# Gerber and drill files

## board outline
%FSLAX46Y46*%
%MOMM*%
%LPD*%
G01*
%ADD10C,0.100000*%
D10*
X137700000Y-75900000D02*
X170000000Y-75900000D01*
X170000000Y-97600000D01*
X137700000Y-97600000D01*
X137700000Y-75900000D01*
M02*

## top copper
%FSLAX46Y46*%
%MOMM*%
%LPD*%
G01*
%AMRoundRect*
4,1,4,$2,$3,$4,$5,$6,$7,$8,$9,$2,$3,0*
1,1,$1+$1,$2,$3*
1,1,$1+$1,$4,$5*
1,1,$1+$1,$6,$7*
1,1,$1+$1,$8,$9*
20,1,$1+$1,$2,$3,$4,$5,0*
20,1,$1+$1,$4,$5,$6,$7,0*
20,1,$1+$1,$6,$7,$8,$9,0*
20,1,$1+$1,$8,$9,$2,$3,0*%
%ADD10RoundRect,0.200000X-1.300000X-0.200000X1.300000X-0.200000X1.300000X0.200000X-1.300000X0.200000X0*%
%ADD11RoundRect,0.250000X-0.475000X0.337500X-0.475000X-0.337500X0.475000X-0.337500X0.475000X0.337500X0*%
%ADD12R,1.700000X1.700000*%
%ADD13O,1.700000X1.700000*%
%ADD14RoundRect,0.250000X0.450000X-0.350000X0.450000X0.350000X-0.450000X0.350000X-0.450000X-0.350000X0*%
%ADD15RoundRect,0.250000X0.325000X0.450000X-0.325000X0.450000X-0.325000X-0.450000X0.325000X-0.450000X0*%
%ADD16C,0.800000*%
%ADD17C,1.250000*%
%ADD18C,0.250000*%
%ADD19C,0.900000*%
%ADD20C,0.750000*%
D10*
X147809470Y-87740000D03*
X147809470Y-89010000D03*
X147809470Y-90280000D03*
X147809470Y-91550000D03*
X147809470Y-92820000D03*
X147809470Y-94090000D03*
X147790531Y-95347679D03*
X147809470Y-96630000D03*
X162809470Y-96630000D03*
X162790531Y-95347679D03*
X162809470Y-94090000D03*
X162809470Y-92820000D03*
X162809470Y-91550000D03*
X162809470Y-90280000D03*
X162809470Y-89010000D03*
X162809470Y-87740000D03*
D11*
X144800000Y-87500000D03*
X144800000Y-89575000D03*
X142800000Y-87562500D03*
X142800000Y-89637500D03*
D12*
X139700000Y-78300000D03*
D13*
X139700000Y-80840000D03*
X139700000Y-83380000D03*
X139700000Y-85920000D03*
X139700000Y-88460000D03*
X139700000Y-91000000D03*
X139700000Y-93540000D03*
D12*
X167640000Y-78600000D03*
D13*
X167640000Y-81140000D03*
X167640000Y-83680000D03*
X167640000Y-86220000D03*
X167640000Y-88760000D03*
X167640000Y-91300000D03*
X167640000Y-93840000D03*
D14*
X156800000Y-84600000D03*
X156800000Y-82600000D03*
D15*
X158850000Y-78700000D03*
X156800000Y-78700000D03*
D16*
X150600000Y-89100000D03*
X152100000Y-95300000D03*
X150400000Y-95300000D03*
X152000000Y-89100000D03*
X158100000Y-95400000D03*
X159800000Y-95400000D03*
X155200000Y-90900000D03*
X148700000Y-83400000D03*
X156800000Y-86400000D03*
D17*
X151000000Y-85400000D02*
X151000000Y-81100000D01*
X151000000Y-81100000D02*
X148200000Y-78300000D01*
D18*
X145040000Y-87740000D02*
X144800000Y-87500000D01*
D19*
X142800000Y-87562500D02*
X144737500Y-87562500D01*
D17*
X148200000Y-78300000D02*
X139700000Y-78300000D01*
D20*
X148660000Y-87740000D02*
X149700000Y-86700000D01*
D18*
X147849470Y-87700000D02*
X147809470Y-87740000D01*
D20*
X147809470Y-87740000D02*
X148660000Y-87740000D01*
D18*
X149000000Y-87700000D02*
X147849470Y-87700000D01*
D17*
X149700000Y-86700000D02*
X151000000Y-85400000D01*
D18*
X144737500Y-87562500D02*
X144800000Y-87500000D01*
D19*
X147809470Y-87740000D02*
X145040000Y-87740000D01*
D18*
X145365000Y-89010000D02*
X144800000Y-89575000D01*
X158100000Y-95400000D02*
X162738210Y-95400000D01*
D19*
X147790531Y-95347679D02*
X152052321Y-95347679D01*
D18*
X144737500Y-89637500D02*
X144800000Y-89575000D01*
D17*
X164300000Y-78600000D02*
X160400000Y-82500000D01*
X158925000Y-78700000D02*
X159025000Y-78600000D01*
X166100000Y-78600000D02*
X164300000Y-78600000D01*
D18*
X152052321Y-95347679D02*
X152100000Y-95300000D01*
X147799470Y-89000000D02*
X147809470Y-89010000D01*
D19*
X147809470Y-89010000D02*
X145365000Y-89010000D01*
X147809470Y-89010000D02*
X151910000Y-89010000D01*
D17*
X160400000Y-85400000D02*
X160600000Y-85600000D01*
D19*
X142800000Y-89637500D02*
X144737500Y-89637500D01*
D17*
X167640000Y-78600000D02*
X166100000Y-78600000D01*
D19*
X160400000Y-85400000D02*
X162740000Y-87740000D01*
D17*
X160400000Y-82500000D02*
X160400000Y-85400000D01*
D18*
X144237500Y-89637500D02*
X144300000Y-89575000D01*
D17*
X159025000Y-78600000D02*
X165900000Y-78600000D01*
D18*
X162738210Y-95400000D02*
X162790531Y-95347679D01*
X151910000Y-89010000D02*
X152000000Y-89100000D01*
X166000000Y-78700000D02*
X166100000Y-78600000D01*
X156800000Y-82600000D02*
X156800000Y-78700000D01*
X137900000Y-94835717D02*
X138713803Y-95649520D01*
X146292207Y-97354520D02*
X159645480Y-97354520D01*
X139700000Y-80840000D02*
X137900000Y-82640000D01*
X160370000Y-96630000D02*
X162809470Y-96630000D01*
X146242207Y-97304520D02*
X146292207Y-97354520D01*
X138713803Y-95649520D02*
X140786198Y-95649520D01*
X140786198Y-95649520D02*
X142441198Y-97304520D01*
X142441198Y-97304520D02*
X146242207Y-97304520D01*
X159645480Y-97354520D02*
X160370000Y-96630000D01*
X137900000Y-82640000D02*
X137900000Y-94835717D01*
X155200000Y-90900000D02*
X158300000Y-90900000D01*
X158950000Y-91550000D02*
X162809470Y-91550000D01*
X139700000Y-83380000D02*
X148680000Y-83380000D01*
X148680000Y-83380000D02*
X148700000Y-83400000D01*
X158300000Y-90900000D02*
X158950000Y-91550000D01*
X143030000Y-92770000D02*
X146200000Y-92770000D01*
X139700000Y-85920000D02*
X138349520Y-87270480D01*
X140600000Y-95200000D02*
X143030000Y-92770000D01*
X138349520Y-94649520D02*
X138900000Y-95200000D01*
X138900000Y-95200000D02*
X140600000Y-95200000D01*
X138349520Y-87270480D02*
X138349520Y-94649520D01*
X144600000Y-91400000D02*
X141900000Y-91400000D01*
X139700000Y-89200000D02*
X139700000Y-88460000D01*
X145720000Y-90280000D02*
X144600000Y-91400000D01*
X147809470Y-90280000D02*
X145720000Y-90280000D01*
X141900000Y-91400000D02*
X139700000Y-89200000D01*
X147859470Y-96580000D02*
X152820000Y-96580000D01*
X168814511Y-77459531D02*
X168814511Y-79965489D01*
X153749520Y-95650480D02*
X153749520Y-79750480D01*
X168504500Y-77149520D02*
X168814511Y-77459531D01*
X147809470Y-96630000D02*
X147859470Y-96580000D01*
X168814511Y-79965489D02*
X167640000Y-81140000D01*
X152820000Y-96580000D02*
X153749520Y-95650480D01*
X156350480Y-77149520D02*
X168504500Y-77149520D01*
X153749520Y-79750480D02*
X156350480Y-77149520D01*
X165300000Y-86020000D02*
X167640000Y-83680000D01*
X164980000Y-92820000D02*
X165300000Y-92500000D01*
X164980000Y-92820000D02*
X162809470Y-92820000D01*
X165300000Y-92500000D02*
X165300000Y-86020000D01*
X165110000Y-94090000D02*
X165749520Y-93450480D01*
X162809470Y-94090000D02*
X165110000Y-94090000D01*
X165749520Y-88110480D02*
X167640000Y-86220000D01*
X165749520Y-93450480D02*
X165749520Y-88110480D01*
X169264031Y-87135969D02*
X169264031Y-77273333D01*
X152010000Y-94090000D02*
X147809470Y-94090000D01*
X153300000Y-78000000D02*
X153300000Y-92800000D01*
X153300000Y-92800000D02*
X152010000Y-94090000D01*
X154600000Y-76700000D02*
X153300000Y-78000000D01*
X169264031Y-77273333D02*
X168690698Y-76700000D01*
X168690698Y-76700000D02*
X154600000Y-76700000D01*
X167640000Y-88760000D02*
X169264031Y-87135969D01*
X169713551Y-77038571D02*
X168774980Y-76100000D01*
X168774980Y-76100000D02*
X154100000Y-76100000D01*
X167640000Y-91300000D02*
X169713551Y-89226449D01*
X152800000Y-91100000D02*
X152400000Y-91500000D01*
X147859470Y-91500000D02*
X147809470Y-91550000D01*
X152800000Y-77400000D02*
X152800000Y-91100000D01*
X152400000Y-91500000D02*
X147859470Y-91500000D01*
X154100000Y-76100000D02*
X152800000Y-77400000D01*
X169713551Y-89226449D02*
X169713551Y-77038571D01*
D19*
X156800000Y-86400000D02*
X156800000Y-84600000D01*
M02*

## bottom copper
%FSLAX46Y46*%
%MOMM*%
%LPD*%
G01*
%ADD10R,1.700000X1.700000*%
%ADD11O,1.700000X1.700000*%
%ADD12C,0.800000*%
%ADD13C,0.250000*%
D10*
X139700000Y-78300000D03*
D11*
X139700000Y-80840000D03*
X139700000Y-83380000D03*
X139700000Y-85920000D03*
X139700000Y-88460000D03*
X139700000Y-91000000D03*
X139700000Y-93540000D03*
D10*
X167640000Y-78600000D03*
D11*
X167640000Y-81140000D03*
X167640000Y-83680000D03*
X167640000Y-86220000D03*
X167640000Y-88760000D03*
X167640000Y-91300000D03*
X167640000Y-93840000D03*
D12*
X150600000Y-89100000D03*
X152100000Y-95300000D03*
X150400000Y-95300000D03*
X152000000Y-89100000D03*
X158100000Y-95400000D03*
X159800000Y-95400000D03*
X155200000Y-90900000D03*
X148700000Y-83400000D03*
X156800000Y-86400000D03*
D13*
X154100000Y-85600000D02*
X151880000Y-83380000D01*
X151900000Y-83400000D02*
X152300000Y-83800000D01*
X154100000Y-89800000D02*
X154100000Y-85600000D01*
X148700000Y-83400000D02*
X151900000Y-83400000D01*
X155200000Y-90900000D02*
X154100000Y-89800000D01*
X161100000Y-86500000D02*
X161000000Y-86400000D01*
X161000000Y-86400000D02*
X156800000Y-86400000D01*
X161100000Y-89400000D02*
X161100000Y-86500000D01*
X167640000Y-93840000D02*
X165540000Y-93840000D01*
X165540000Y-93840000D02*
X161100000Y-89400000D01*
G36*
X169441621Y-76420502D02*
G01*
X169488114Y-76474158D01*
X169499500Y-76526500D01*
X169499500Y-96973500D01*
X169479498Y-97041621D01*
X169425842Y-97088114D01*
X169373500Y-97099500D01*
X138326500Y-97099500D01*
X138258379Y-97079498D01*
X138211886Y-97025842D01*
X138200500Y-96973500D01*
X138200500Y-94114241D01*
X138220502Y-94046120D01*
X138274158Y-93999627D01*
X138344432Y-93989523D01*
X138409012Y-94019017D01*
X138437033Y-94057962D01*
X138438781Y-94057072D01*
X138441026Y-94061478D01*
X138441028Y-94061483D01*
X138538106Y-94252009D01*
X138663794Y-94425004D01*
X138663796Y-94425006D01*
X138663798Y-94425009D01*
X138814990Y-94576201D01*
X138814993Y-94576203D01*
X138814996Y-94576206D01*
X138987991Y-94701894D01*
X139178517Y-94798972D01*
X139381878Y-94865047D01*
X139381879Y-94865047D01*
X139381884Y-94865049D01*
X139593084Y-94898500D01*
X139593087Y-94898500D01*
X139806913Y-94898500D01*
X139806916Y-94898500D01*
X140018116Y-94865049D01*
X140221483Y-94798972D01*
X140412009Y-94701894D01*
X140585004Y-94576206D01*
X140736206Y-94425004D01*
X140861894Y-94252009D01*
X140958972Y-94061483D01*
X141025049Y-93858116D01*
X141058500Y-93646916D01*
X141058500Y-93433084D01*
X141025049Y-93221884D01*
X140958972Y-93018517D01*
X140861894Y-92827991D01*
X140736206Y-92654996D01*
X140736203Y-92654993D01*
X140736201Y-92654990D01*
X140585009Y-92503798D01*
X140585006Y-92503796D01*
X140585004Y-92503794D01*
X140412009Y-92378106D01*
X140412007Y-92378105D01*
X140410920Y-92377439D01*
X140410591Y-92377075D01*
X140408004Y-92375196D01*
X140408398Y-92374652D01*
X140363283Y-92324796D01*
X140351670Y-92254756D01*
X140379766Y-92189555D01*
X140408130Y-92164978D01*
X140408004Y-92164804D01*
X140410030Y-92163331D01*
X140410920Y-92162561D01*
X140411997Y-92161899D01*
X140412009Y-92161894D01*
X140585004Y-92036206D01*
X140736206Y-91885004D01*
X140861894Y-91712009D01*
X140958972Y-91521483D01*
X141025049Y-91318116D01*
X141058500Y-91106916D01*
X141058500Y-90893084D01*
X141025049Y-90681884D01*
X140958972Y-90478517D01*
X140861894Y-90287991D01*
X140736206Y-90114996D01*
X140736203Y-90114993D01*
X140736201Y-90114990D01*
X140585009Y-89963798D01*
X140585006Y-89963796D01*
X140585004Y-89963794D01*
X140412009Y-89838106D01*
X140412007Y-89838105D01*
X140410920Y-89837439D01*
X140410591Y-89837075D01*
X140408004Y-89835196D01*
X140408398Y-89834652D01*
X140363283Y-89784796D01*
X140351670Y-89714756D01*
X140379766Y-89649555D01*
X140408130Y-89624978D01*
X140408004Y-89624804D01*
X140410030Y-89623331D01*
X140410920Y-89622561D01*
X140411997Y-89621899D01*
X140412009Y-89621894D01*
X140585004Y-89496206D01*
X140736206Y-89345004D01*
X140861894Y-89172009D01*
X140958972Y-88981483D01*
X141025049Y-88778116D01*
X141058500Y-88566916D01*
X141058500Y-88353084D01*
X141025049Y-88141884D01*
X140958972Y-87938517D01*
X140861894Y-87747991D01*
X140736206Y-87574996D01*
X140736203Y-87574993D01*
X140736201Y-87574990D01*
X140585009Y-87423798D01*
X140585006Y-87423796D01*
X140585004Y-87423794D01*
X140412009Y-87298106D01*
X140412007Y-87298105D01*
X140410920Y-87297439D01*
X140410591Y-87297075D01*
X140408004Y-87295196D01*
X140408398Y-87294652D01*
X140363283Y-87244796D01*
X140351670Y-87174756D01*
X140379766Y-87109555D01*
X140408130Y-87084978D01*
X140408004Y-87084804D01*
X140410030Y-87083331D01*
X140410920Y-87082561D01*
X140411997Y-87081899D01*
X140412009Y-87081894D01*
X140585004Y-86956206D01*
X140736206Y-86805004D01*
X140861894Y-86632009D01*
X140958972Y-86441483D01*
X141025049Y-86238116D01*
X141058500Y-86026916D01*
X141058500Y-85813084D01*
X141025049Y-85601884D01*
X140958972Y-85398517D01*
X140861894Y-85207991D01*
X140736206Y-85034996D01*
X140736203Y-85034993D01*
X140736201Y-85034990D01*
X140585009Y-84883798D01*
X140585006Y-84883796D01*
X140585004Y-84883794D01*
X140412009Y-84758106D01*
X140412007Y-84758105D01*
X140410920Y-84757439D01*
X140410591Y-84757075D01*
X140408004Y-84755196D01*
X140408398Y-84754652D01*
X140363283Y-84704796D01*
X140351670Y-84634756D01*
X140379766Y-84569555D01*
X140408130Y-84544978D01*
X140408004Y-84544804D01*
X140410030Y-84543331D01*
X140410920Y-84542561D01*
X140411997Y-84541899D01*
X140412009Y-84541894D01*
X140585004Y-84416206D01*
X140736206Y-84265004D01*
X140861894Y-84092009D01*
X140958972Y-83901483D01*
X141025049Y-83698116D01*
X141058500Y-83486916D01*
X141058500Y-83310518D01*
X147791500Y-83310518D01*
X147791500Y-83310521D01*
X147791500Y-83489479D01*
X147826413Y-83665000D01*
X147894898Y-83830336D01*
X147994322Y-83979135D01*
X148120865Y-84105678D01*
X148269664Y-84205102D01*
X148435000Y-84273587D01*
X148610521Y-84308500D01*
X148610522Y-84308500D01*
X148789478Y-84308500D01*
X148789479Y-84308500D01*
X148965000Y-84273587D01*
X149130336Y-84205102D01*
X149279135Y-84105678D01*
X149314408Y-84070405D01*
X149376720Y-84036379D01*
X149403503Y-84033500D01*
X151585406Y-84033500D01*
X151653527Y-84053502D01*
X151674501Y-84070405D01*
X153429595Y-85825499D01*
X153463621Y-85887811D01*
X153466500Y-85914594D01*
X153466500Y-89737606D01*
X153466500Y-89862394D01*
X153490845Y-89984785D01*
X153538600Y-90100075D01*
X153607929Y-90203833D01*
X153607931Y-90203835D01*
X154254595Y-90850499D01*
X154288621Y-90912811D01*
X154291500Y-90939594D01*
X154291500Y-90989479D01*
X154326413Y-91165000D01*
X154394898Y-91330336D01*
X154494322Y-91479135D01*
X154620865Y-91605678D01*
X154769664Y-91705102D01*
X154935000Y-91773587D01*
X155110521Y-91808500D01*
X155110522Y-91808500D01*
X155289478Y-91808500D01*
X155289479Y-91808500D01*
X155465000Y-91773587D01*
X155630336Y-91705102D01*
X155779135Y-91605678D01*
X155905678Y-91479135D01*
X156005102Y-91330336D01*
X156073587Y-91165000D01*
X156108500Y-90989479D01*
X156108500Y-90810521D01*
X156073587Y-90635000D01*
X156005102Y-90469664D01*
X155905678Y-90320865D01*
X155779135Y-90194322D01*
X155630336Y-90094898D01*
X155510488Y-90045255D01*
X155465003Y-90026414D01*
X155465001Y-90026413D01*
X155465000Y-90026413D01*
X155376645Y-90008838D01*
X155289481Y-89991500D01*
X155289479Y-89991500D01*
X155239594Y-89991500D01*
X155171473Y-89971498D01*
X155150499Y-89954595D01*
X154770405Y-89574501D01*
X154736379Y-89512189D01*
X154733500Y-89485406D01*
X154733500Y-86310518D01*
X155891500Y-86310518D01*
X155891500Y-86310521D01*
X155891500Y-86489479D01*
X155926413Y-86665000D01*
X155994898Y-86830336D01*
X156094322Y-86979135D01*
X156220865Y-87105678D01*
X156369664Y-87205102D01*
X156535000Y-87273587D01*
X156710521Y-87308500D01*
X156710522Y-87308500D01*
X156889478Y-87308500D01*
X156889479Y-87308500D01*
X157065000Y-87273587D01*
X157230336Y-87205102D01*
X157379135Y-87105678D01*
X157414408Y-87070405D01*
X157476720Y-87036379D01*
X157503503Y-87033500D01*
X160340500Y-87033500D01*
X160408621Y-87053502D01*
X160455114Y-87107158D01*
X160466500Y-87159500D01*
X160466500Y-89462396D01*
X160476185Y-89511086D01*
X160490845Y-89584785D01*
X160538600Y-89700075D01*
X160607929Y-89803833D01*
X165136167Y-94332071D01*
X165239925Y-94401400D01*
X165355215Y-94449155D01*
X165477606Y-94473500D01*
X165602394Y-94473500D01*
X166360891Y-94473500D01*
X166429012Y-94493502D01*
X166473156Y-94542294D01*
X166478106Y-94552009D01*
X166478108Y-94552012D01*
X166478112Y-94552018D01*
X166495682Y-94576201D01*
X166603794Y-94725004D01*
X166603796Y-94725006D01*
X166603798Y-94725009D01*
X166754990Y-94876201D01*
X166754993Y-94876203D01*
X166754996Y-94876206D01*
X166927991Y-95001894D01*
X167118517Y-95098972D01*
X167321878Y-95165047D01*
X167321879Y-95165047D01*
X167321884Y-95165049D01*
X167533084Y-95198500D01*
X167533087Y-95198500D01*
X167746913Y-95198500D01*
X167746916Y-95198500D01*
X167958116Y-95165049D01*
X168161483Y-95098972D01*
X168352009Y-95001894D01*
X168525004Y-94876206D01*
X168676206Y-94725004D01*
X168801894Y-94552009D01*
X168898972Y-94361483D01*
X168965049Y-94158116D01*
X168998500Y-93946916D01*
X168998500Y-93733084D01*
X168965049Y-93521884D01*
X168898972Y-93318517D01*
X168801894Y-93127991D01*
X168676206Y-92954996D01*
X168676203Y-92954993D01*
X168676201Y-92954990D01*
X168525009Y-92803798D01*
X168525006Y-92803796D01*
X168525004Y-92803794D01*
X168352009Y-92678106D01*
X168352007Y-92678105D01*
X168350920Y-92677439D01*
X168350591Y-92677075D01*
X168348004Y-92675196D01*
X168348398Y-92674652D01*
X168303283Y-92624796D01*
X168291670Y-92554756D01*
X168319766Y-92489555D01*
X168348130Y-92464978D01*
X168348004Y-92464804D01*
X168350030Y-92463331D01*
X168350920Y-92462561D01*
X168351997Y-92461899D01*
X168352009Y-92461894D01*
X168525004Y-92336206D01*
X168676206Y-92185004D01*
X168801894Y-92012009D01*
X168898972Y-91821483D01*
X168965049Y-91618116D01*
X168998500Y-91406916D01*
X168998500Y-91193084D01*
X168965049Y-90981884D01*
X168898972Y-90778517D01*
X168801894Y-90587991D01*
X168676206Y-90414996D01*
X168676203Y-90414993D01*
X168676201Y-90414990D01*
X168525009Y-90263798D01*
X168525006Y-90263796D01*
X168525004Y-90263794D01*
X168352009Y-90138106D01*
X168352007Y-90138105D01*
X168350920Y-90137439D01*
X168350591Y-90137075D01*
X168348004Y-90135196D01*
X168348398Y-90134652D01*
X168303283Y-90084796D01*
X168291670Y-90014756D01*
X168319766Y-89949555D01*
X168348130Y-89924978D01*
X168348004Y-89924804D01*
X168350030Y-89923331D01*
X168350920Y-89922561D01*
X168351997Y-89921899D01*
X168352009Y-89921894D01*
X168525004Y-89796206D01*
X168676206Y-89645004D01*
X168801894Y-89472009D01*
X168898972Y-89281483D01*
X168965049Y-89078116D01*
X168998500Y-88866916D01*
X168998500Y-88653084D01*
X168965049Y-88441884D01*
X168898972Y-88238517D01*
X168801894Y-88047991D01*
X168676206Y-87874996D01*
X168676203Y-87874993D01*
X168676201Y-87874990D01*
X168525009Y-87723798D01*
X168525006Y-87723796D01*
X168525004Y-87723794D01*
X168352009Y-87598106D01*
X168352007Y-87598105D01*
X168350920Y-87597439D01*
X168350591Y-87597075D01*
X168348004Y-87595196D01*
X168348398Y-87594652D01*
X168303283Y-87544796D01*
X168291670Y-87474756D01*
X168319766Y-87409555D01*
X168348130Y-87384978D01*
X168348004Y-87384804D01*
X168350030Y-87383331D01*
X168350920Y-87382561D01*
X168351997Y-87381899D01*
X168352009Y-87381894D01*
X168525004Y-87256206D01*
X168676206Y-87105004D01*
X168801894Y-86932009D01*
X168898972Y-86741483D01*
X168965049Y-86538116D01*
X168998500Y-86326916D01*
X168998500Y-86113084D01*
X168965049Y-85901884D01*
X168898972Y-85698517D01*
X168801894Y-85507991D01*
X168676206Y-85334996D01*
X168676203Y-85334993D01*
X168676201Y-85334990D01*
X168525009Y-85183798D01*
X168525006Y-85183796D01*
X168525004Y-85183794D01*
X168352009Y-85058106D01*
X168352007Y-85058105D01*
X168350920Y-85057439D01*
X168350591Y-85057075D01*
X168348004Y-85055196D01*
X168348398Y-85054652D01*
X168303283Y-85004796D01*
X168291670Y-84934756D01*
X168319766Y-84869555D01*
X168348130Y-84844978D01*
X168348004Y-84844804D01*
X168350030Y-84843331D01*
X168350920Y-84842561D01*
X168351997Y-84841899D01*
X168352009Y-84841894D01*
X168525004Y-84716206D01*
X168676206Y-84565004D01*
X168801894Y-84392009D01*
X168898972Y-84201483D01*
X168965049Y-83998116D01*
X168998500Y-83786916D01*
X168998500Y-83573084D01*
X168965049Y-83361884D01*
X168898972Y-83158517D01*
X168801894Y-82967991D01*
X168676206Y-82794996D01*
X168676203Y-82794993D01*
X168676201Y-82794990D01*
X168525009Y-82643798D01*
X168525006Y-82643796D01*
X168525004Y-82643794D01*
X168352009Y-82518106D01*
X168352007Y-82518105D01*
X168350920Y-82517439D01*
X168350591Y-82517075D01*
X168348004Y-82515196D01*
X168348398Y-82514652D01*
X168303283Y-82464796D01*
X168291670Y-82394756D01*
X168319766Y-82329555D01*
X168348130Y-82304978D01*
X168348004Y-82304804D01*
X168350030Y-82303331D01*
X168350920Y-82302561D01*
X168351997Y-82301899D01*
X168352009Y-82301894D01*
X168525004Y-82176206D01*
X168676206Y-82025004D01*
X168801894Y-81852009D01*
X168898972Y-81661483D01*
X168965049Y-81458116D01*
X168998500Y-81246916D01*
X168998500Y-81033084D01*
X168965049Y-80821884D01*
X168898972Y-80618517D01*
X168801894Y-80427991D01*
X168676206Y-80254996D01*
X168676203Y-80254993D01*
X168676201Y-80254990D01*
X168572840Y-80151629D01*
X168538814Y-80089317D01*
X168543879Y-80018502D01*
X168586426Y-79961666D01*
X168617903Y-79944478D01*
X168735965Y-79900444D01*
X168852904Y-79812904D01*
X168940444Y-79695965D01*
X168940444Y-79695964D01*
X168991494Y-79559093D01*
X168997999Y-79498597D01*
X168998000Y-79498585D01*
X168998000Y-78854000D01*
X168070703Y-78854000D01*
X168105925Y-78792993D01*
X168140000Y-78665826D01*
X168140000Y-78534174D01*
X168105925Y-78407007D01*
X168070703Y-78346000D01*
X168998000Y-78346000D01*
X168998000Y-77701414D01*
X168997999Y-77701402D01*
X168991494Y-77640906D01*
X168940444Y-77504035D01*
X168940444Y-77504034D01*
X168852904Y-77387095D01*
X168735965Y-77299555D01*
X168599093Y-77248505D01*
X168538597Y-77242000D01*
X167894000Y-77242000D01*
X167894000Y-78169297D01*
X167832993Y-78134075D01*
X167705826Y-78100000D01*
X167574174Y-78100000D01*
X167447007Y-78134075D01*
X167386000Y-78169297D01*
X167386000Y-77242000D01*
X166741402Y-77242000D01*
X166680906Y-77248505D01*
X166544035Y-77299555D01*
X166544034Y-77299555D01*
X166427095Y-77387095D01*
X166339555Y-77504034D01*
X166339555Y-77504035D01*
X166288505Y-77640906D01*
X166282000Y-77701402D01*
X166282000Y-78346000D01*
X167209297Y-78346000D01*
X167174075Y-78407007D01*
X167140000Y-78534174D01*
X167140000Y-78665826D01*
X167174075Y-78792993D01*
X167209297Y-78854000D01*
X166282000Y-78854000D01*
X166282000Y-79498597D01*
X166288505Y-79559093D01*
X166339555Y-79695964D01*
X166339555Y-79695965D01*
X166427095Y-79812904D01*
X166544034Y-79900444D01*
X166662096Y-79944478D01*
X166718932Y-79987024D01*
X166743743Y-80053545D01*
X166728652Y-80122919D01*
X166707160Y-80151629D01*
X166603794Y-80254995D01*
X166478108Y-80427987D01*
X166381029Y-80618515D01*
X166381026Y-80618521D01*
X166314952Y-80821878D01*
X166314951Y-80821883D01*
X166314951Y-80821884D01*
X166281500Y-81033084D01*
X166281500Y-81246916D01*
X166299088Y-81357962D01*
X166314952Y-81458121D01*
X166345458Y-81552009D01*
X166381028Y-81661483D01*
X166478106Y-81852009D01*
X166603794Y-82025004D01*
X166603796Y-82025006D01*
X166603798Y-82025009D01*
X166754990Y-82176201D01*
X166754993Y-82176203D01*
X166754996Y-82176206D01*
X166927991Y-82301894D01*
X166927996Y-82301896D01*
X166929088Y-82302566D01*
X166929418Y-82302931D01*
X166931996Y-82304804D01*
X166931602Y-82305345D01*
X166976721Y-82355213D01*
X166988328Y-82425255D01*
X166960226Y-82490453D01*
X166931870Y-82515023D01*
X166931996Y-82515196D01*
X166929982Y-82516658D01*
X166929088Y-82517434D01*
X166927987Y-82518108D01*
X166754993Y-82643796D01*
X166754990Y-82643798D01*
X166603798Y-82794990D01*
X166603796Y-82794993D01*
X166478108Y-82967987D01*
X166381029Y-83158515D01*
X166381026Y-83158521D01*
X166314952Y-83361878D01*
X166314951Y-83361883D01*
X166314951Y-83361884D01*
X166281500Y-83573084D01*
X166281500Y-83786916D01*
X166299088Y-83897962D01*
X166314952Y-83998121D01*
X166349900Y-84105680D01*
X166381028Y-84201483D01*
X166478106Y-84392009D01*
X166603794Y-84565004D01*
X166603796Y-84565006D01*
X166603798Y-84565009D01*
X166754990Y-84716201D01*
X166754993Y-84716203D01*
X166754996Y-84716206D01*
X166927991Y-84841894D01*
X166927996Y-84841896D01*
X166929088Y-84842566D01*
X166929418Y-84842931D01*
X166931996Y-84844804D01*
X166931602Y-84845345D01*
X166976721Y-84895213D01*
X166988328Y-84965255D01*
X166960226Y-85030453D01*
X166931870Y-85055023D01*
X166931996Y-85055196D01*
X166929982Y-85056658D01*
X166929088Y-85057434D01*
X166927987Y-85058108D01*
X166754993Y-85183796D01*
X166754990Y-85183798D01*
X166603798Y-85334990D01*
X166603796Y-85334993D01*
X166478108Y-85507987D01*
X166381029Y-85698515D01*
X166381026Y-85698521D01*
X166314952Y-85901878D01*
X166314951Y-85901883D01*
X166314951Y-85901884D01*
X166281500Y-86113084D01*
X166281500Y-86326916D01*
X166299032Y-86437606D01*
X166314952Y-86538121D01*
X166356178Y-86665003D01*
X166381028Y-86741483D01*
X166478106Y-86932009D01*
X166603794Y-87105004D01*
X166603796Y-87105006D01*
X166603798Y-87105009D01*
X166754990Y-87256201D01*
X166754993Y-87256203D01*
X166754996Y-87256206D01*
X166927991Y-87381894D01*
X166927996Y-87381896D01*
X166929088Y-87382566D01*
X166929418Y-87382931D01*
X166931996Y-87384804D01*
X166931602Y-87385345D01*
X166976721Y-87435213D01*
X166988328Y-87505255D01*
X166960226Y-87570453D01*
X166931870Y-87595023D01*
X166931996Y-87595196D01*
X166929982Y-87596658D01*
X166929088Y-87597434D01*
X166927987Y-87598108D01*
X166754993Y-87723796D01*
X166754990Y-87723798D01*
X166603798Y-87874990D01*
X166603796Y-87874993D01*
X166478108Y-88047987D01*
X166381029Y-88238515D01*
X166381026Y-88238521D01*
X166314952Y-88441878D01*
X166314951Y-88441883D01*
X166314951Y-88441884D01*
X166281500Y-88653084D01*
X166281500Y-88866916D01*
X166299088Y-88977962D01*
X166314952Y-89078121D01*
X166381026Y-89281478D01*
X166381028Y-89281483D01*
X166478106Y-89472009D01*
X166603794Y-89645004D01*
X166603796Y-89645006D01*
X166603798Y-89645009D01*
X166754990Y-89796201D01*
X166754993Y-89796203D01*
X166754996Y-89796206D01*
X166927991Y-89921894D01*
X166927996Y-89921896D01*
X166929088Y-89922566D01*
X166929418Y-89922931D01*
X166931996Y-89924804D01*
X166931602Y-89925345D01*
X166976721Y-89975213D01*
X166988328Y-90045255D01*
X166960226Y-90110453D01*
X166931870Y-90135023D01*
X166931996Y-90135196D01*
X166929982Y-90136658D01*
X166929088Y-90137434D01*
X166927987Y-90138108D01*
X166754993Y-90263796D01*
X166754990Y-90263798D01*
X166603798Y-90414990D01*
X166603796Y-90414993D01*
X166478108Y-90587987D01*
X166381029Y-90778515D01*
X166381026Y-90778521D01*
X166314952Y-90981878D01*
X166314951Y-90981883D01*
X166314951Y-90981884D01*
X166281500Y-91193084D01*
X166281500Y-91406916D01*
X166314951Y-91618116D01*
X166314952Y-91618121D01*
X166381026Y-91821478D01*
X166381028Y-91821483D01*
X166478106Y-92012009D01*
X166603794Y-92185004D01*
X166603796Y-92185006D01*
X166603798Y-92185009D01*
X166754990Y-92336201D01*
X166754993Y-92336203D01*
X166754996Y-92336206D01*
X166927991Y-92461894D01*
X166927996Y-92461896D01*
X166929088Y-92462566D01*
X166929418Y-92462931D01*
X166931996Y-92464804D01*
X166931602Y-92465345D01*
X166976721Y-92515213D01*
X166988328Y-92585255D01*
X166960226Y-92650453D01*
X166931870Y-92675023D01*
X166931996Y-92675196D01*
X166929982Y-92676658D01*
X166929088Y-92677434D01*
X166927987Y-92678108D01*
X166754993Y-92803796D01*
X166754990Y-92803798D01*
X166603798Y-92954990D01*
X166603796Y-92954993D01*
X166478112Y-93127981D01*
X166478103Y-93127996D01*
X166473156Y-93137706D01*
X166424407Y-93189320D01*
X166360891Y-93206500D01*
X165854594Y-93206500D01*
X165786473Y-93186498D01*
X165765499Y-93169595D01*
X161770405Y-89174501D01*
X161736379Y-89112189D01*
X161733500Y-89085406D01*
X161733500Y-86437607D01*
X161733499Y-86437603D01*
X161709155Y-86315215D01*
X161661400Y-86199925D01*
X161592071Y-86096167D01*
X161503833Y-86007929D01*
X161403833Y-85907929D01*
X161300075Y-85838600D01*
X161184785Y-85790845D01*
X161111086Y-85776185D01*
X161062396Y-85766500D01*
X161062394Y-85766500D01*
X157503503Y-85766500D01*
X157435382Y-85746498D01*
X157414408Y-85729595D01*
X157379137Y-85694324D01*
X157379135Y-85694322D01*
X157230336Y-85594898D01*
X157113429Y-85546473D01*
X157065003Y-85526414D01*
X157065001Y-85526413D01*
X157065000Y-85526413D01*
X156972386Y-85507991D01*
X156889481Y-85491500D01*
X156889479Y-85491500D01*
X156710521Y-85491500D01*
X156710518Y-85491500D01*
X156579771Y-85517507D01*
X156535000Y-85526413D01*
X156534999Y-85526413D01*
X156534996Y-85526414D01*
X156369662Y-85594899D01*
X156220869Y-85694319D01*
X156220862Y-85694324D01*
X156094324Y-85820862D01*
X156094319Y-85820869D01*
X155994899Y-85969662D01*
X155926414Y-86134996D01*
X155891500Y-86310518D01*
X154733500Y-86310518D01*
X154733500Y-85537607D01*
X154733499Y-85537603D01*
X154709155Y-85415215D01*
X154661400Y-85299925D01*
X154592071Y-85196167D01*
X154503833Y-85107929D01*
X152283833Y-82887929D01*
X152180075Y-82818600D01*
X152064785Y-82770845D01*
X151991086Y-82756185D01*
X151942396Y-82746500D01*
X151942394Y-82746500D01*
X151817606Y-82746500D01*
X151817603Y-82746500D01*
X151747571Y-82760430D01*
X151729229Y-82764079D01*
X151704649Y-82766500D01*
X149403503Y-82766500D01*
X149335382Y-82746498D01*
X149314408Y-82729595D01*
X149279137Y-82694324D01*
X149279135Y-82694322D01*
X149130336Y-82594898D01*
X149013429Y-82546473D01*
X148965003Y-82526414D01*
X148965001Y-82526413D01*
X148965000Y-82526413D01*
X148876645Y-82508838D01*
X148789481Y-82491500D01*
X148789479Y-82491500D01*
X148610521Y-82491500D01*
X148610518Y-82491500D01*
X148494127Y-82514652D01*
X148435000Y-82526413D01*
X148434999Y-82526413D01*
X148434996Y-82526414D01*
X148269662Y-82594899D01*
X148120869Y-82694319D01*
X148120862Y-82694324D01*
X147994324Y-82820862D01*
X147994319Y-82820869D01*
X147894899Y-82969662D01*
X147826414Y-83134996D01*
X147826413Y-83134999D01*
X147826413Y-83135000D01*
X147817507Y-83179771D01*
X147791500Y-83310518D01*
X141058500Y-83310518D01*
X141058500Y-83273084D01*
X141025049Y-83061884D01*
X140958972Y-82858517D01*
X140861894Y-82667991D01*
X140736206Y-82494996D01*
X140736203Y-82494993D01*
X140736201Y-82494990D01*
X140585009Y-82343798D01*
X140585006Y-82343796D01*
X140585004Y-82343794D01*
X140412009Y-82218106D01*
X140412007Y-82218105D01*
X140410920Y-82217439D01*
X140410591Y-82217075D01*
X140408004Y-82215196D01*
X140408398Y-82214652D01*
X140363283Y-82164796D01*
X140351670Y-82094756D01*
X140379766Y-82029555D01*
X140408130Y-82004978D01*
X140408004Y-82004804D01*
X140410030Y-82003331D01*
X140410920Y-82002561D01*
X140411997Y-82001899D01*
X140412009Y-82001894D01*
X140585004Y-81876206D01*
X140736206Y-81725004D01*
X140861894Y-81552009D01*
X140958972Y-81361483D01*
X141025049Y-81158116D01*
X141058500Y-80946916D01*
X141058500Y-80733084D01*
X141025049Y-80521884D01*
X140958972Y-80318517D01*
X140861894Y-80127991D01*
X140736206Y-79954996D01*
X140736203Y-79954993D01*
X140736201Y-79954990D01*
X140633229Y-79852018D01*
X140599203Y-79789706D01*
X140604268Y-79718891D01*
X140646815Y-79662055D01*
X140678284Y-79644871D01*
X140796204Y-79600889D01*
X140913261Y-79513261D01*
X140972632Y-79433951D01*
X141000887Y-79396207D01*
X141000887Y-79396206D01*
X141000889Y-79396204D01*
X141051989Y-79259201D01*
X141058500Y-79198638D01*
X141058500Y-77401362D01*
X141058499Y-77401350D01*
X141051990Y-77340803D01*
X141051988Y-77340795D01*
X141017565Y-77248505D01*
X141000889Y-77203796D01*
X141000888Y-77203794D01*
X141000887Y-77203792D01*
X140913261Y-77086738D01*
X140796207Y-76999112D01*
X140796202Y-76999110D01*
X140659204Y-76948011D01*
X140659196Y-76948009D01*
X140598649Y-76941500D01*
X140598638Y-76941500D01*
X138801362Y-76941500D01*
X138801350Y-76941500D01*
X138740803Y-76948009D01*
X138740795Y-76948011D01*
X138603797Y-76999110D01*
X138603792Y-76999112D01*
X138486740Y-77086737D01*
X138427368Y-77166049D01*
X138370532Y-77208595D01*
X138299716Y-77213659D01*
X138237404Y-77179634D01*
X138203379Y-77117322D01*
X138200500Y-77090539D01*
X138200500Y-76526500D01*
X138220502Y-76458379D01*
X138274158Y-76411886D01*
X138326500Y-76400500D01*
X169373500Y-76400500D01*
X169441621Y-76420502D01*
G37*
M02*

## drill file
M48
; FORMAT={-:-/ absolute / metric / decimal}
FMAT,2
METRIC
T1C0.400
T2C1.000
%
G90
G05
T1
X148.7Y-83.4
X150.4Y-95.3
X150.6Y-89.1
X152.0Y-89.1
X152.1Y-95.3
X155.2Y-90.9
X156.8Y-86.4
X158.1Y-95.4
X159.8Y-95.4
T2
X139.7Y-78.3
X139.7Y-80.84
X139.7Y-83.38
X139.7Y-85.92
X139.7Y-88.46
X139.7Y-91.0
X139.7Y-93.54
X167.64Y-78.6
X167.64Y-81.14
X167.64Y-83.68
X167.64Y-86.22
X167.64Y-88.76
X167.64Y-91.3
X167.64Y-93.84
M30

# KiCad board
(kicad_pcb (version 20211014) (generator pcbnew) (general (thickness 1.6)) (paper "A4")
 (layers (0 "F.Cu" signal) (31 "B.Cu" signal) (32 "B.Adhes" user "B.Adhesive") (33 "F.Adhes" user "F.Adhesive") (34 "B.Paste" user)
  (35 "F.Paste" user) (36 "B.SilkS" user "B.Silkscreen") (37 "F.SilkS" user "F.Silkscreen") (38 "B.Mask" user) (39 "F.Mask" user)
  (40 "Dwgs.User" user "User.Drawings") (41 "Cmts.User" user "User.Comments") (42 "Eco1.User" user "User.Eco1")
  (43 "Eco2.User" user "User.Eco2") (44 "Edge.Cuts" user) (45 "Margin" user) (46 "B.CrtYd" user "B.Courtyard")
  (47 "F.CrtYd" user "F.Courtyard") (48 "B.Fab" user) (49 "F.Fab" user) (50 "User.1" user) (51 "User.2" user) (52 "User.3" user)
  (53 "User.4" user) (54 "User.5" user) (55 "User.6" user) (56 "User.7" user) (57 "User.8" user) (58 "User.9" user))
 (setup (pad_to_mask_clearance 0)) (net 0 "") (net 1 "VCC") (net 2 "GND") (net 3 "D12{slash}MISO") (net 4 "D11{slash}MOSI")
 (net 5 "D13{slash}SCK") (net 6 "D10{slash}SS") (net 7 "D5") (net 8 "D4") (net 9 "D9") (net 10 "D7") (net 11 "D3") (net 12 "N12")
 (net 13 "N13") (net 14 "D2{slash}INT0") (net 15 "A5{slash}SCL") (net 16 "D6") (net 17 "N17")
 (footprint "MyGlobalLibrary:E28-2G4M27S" (layer "F.Cu") (at 147.80947 87.74)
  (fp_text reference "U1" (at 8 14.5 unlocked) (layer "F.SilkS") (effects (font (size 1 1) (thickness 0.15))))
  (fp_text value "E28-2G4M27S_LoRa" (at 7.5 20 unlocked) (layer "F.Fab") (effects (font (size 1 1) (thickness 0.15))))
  (pad "1" smd roundrect (at 0 0) (size 3 0.8) (layers "F.Cu" "F.Paste" "F.Mask") (roundrect_rratio 0.25) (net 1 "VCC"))
  (pad "2" smd roundrect (at 0 1.27) (size 3 0.8) (layers "F.Cu" "F.Paste" "F.Mask") (roundrect_rratio 0.25) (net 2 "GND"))
  (pad "3" smd roundrect (at 0 2.54) (size 3 0.8) (layers "F.Cu" "F.Paste" "F.Mask") (roundrect_rratio 0.25) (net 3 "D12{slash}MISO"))
  (pad "4" smd roundrect (at 0 3.81) (size 3 0.8) (layers "F.Cu" "F.Paste" "F.Mask") (roundrect_rratio 0.25) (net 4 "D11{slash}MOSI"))
  (pad "5" smd roundrect (at 0 5.08) (size 3 0.8) (layers "F.Cu" "F.Paste" "F.Mask") (roundrect_rratio 0.25) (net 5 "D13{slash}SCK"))
  (pad "6" smd roundrect (at 0 6.35) (size 3 0.8) (layers "F.Cu" "F.Paste" "F.Mask") (roundrect_rratio 0.25) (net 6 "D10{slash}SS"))
  (pad "7" smd roundrect (at -0.018939 7.607679) (size 3 0.8) (layers "F.Cu" "F.Paste" "F.Mask") (roundrect_rratio 0.25) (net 2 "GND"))
  (pad "8" smd roundrect (at 0 8.89) (size 3 0.8) (layers "F.Cu" "F.Paste" "F.Mask") (roundrect_rratio 0.25) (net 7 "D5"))
  (pad "9" smd roundrect (at 15 8.89) (size 3 0.8) (layers "F.Cu" "F.Paste" "F.Mask") (roundrect_rratio 0.25) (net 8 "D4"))
  (pad "10" smd roundrect (at 14.981061 7.607679) (size 3 0.8) (layers "F.Cu" "F.Paste" "F.Mask") (roundrect_rratio 0.25) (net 2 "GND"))
  (pad "11" smd roundrect (at 15 6.35) (size 3 0.8) (layers "F.Cu" "F.Paste" "F.Mask") (roundrect_rratio 0.25) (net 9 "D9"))
  (pad "12" smd roundrect (at 15 5.08) (size 3 0.8) (layers "F.Cu" "F.Paste" "F.Mask") (roundrect_rratio 0.25) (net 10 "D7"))
  (pad "13" smd roundrect (at 15 3.81) (size 3 0.8) (layers "F.Cu" "F.Paste" "F.Mask") (roundrect_rratio 0.25) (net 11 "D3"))
  (pad "14" smd roundrect (at 15 2.54) (size 3 0.8) (layers "F.Cu" "F.Paste" "F.Mask") (roundrect_rratio 0.25) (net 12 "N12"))
  (pad "15" smd roundrect (at 15 1.27) (size 3 0.8) (layers "F.Cu" "F.Paste" "F.Mask") (roundrect_rratio 0.25) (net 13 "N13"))
  (pad "16" smd roundrect (at 15 0) (size 3 0.8) (layers "F.Cu" "F.Paste" "F.Mask") (roundrect_rratio 0.25) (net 2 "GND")))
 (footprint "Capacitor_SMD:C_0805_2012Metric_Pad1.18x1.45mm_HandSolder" (layer "F.Cu") (at 144.8 88.5375 -90)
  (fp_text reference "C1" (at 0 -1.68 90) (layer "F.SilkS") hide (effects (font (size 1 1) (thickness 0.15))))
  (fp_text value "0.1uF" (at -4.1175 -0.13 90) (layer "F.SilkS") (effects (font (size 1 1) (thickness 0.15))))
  (pad "1" smd roundrect (at -1.0375 0 270) (size 1.175 1.45) (layers "F.Cu" "F.Paste" "F.Mask") (roundrect_rratio 0.2127659574)
   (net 1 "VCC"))
  (pad "2" smd roundrect (at 1.0375 0 270) (size 1.175 1.45) (layers "F.Cu" "F.Paste" "F.Mask") (roundrect_rratio 0.2127659574)
   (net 2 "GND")))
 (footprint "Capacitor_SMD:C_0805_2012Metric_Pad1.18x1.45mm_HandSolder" (layer "F.Cu") (at 142.8 88.6 -90)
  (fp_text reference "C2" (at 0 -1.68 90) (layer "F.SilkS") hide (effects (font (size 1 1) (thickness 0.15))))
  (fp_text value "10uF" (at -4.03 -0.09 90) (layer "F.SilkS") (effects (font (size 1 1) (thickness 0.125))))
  (pad "1" smd roundrect (at -1.0375 0 270) (size 1.175 1.45) (layers "F.Cu" "F.Paste" "F.Mask") (roundrect_rratio 0.2127659574)
   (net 1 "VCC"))
  (pad "2" smd roundrect (at 1.0375 0 270) (size 1.175 1.45) (layers "F.Cu" "F.Paste" "F.Mask") (roundrect_rratio 0.2127659574)
   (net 2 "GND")))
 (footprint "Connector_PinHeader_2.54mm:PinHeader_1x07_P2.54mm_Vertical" (layer "F.Cu") (at 139.7 78.3)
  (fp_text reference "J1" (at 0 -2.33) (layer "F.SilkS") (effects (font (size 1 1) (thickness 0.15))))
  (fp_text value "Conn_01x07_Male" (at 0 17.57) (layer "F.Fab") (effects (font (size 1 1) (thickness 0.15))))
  (pad "1" thru_hole rect (at 0 0) (size 1.7 1.7) (drill 1) (layers *.Cu *.Mask) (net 1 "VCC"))
  (pad "2" thru_hole oval (at 0 2.54) (size 1.7 1.7) (drill 1) (layers *.Cu *.Mask) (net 8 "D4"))
  (pad "3" thru_hole oval (at 0 5.08) (size 1.7 1.7) (drill 1) (layers *.Cu *.Mask) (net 11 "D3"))
  (pad "4" thru_hole oval (at 0 7.62) (size 1.7 1.7) (drill 1) (layers *.Cu *.Mask) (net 5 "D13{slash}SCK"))
  (pad "5" thru_hole oval (at 0 10.16) (size 1.7 1.7) (drill 1) (layers *.Cu *.Mask) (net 3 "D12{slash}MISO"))
  (pad "6" thru_hole oval (at 0 12.7) (size 1.7 1.7) (drill 1) (layers *.Cu *.Mask) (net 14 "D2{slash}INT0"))
  (pad "7" thru_hole oval (at 0 15.24) (size 1.7 1.7) (drill 1) (layers *.Cu *.Mask) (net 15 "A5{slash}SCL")))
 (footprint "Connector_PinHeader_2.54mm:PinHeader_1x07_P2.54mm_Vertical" (layer "F.Cu") (at 167.64 78.6)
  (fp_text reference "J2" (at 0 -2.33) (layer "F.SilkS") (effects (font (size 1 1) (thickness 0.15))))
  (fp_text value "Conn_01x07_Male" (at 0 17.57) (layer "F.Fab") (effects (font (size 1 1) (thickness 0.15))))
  (pad "1" thru_hole rect (at 0 0) (size 1.7 1.7) (drill 1) (layers *.Cu *.Mask) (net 2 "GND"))
  (pad "2" thru_hole oval (at 0 2.54) (size 1.7 1.7) (drill 1) (layers *.Cu *.Mask) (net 7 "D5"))
  (pad "3" thru_hole oval (at 0 5.08) (size 1.7 1.7) (drill 1) (layers *.Cu *.Mask) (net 10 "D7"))
  (pad "4" thru_hole oval (at 0 7.62) (size 1.7 1.7) (drill 1) (layers *.Cu *.Mask) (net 9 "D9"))
  (pad "5" thru_hole oval (at 0 10.16) (size 1.7 1.7) (drill 1) (layers *.Cu *.Mask) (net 6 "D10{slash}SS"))
  (pad "6" thru_hole oval (at 0 12.7) (size 1.7 1.7) (drill 1) (layers *.Cu *.Mask) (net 4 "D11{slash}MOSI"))
  (pad "7" thru_hole oval (at 0 15.24) (size 1.7 1.7) (drill 1) (layers *.Cu *.Mask) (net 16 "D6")))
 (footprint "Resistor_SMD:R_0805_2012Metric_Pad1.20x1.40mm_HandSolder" (layer "F.Cu") (at 156.8 83.6 90)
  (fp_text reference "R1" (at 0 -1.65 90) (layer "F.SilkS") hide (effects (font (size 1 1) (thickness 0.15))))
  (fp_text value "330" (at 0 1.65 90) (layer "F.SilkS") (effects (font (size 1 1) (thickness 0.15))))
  (pad "1" smd roundrect (at -1 0 90) (size 1.2 1.4) (layers "F.Cu" "F.Paste" "F.Mask") (roundrect_rratio 0.2083333333) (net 16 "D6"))
  (pad "2" smd roundrect (at 1 0 90) (size 1.2 1.4) (layers "F.Cu" "F.Paste" "F.Mask") (roundrect_rratio 0.2083333333) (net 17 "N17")))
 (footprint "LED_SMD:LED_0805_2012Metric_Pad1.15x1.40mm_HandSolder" (layer "F.Cu") (at 157.825 78.7 180)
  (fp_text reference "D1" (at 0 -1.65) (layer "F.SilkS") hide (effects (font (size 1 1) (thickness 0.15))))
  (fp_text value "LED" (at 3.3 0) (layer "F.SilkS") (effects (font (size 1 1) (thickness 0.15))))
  (pad "1" smd roundrect (at -1.025 0 180) (size 1.15 1.4) (layers "F.Cu" "F.Paste" "F.Mask") (roundrect_rratio 0.2173913043) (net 2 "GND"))
  (pad "2" smd roundrect (at 1.025 0 180) (size 1.15 1.4) (layers "F.Cu" "F.Paste" "F.Mask") (roundrect_rratio 0.2173913043) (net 17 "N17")))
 (gr_rect (start 137.7 75.9) (end 170 97.6) (layer "Edge.Cuts") (width 0.1) (fill none))
 (segment (start 151 85.4) (end 151 81.1) (width 1.25) (layer "F.Cu") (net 1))
 (segment (start 151 81.1) (end 148.2 78.3) (width 1.25) (layer "F.Cu") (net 1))
 (segment (start 145.04 87.74) (end 144.8 87.5) (width 0.25) (layer "F.Cu") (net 1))
 (segment (start 142.8 87.5625) (end 144.7375 87.5625) (width 0.9) (layer "F.Cu") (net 1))
 (segment (start 148.2 78.3) (end 139.7 78.3) (width 1.25) (layer "F.Cu") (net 1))
 (segment (start 148.66 87.74) (end 149.7 86.7) (width 0.75) (layer "F.Cu") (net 1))
 (segment (start 147.84947 87.7) (end 147.80947 87.74) (width 0.25) (layer "F.Cu") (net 1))
 (segment (start 147.80947 87.74) (end 148.66 87.74) (width 0.75) (layer "F.Cu") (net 1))
 (segment (start 149 87.7) (end 147.84947 87.7) (width 0.25) (layer "F.Cu") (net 1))
 (segment (start 149.7 86.7) (end 151 85.4) (width 1.25) (layer "F.Cu") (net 1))
 (segment (start 144.7375 87.5625) (end 144.8 87.5) (width 0.25) (layer "F.Cu") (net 1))
 (segment (start 147.80947 87.74) (end 145.04 87.74) (width 0.9) (layer "F.Cu") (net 1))
 (segment (start 145.365 89.01) (end 144.8 89.575) (width 0.25) (layer "F.Cu") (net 2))
 (segment (start 158.1 95.4) (end 162.73821 95.4) (width 0.25) (layer "F.Cu") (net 2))
 (segment (start 147.790531 95.347679) (end 152.052321 95.347679) (width 0.9) (layer "F.Cu") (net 2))
 (segment (start 144.7375 89.6375) (end 144.8 89.575) (width 0.25) (layer "F.Cu") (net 2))
 (segment (start 164.3 78.6) (end 160.4 82.5) (width 1.25) (layer "F.Cu") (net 2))
 (segment (start 158.925 78.7) (end 159.025 78.6) (width 1.25) (layer "F.Cu") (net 2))
 (segment (start 166.1 78.6) (end 164.3 78.6) (width 1.25) (layer "F.Cu") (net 2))
 (segment (start 152.052321 95.347679) (end 152.1 95.3) (width 0.25) (layer "F.Cu") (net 2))
 (segment (start 147.79947 89) (end 147.80947 89.01) (width 0.25) (layer "F.Cu") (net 2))
 (segment (start 147.80947 89.01) (end 145.365 89.01) (width 0.9) (layer "F.Cu") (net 2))
 (segment (start 147.80947 89.01) (end 151.91 89.01) (width 0.9) (layer "F.Cu") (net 2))
 (segment (start 160.4 85.4) (end 160.6 85.6) (width 1.25) (layer "F.Cu") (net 2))
 (segment (start 142.8 89.6375) (end 144.7375 89.6375) (width 0.9) (layer "F.Cu") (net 2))
 (segment (start 167.64 78.6) (end 166.1 78.6) (width 1.25) (layer "F.Cu") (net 2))
 (segment (start 160.4 85.4) (end 162.74 87.74) (width 0.9) (layer "F.Cu") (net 2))
 (segment (start 160.4 82.5) (end 160.4 85.4) (width 1.25) (layer "F.Cu") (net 2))
 (segment (start 144.2375 89.6375) (end 144.3 89.575) (width 0.25) (layer "F.Cu") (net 2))
 (segment (start 159.025 78.6) (end 165.9 78.6) (width 1.25) (layer "F.Cu") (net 2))
 (segment (start 162.73821 95.4) (end 162.790531 95.347679) (width 0.25) (layer "F.Cu") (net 2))
 (segment (start 151.91 89.01) (end 152 89.1) (width 0.25) (layer "F.Cu") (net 2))
 (segment (start 166 78.7) (end 166.1 78.6) (width 0.25) (layer "F.Cu") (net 2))
 (via (at 150.6 89.1) (size 0.8) (drill 0.4) (layers "F.Cu" "B.Cu") (free) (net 2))
 (via (at 152.1 95.3) (size 0.8) (drill 0.4) (layers "F.Cu" "B.Cu") (free) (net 2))
 (via (at 150.4 95.3) (size 0.8) (drill 0.4) (layers "F.Cu" "B.Cu") (free) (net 2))
 (via (at 152 89.1) (size 0.8) (drill 0.4) (layers "F.Cu" "B.Cu") (free) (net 2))
 (via (at 158.1 95.4) (size 0.8) (drill 0.4) (layers "F.Cu" "B.Cu") (free) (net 2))
 (via (at 159.8 95.4) (size 0.8) (drill 0.4) (layers "F.Cu" "B.Cu") (free) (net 2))
 (segment (start 156.8 82.6) (end 156.8 78.7) (width 0.25) (layer "F.Cu") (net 17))
 (segment (start 137.9 94.835717) (end 138.713803 95.64952) (width 0.25) (layer "F.Cu") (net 8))
 (segment (start 146.292207 97.35452) (end 159.64548 97.35452) (width 0.25) (layer "F.Cu") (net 8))
 (segment (start 139.7 80.84) (end 137.9 82.64) (width 0.25) (layer "F.Cu") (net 8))
 (segment (start 160.37 96.63) (end 162.80947 96.63) (width 0.25) (layer "F.Cu") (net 8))
 (segment (start 146.242207 97.30452) (end 146.292207 97.35452) (width 0.25) (layer "F.Cu") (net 8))
 (segment (start 138.713803 95.64952) (end 140.786198 95.64952) (width 0.25) (layer "F.Cu") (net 8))
 (segment (start 140.786198 95.64952) (end 142.441198 97.30452) (width 0.25) (layer "F.Cu") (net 8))
 (segment (start 142.441198 97.30452) (end 146.242207 97.30452) (width 0.25) (layer "F.Cu") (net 8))
 (segment (start 159.64548 97.35452) (end 160.37 96.63) (width 0.25) (layer "F.Cu") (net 8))
 (segment (start 137.9 82.64) (end 137.9 94.835717) (width 0.25) (layer "F.Cu") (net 8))
 (segment (start 155.2 90.9) (end 158.3 90.9) (width 0.25) (layer "F.Cu") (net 11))
 (segment (start 158.95 91.55) (end 162.80947 91.55) (width 0.25) (layer "F.Cu") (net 11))
 (segment (start 139.7 83.38) (end 148.68 83.38) (width 0.25) (layer "F.Cu") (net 11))
 (segment (start 148.68 83.38) (end 148.7 83.4) (width 0.25) (layer "F.Cu") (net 11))
 (segment (start 158.3 90.9) (end 158.95 91.55) (width 0.25) (layer "F.Cu") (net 11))
 (via (at 155.2 90.9) (size 0.8) (drill 0.4) (layers "F.Cu" "B.Cu") (free) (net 11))
 (via (at 148.7 83.4) (size 0.8) (drill 0.4) (layers "F.Cu" "B.Cu") (free) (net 11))
 (segment (start 154.1 85.6) (end 151.88 83.38) (width 0.25) (layer "B.Cu") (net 11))
 (segment (start 151.9 83.4) (end 152.3 83.8) (width 0.25) (layer "B.Cu") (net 11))
 (segment (start 154.1 89.8) (end 154.1 85.6) (width 0.25) (layer "B.Cu") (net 11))
 (segment (start 148.7 83.4) (end 151.9 83.4) (width 0.25) (layer "B.Cu") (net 11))
 (segment (start 155.2 90.9) (end 154.1 89.8) (width 0.25) (layer "B.Cu") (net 11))
 (segment (start 143.03 92.77) (end 146.2 92.77) (width 0.25) (layer "F.Cu") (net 5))
 (segment (start 139.7 85.92) (end 138.34952 87.27048) (width 0.25) (layer "F.Cu") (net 5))
 (segment (start 140.6 95.2) (end 143.03 92.77) (width 0.25) (layer "F.Cu") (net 5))
 (segment (start 138.34952 94.64952) (end 138.9 95.2) (width 0.25) (layer "F.Cu") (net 5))
 (segment (start 138.9 95.2) (end 140.6 95.2) (width 0.25) (layer "F.Cu") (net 5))
 (segment (start 138.34952 87.27048) (end 138.34952 94.64952) (width 0.25) (layer "F.Cu") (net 5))
 (segment (start 144.6 91.4) (end 141.9 91.4) (width 0.25) (layer "F.Cu") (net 3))
 (segment (start 139.7 89.2) (end 139.7 88.46) (width 0.25) (layer "F.Cu") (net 3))
 (segment (start 145.72 90.28) (end 144.6 91.4) (width 0.25) (layer "F.Cu") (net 3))
 (segment (start 147.80947 90.28) (end 145.72 90.28) (width 0.25) (layer "F.Cu") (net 3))
 (segment (start 141.9 91.4) (end 139.7 89.2) (width 0.25) (layer "F.Cu") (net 3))
 (segment (start 147.85947 96.58) (end 152.82 96.58) (width 0.25) (layer "F.Cu") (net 7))
 (segment (start 168.814511 77.459531) (end 168.814511 79.965489) (width 0.25) (layer "F.Cu") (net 7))
 (segment (start 153.74952 95.65048) (end 153.74952 79.75048) (width 0.25) (layer "F.Cu") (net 7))
 (segment (start 168.5045 77.14952) (end 168.814511 77.459531) (width 0.25) (layer "F.Cu") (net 7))
 (segment (start 147.80947 96.63) (end 147.85947 96.58) (width 0.25) (layer "F.Cu") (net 7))
 (segment (start 168.814511 79.965489) (end 167.64 81.14) (width 0.25) (layer "F.Cu") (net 7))
 (segment (start 152.82 96.58) (end 153.74952 95.65048) (width 0.25) (layer "F.Cu") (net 7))
 (segment (start 156.35048 77.14952) (end 168.5045 77.14952) (width 0.25) (layer "F.Cu") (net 7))
 (segment (start 153.74952 79.75048) (end 156.35048 77.14952) (width 0.25) (layer "F.Cu") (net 7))
 (segment (start 165.3 86.02) (end 167.64 83.68) (width 0.25) (layer "F.Cu") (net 10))
 (segment (start 164.98 92.82) (end 165.3 92.5) (width 0.25) (layer "F.Cu") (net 10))
 (segment (start 164.98 92.82) (end 162.80947 92.82) (width 0.25) (layer "F.Cu") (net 10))
 (segment (start 165.3 92.5) (end 165.3 86.02) (width 0.25) (layer "F.Cu") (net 10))
 (segment (start 165.11 94.09) (end 165.74952 93.45048) (width 0.25) (layer "F.Cu") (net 9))
 (segment (start 162.80947 94.09) (end 165.11 94.09) (width 0.25) (layer "F.Cu") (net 9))
 (segment (start 165.74952 88.11048) (end 167.64 86.22) (width 0.25) (layer "F.Cu") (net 9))
 (segment (start 165.74952 93.45048) (end 165.74952 88.11048) (width 0.25) (layer "F.Cu") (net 9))
 (segment (start 169.264031 87.135969) (end 169.264031 77.273333) (width 0.25) (layer "F.Cu") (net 6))
 (segment (start 152.01 94.09) (end 147.80947 94.09) (width 0.25) (layer "F.Cu") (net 6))
 (segment (start 153.3 78) (end 153.3 92.8) (width 0.25) (layer "F.Cu") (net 6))
 (segment (start 153.3 92.8) (end 152.01 94.09) (width 0.25) (layer "F.Cu") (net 6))
 (segment (start 154.6 76.7) (end 153.3 78) (width 0.25) (layer "F.Cu") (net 6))
 (segment (start 169.264031 77.273333) (end 168.690698 76.7) (width 0.25) (layer "F.Cu") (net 6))
 (segment (start 168.690698 76.7) (end 154.6 76.7) (width 0.25) (layer "F.Cu") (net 6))
 (segment (start 167.64 88.76) (end 169.264031 87.135969) (width 0.25) (layer "F.Cu") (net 6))
 (segment (start 169.713551 77.038571) (end 168.77498 76.1) (width 0.25) (layer "F.Cu") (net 4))
 (segment (start 168.77498 76.1) (end 154.1 76.1) (width 0.25) (layer "F.Cu") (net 4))
 (segment (start 167.64 91.3) (end 169.713551 89.226449) (width 0.25) (layer "F.Cu") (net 4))
 (segment (start 152.8 91.1) (end 152.4 91.5) (width 0.25) (layer "F.Cu") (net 4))
 (segment (start 147.85947 91.5) (end 147.80947 91.55) (width 0.25) (layer "F.Cu") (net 4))
 (segment (start 152.8 77.4) (end 152.8 91.1) (width 0.25) (layer "F.Cu") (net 4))
 (segment (start 152.4 91.5) (end 147.85947 91.5) (width 0.25) (layer "F.Cu") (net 4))
 (segment (start 154.1 76.1) (end 152.8 77.4) (width 0.25) (layer "F.Cu") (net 4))
 (segment (start 169.713551 89.226449) (end 169.713551 77.038571) (width 0.25) (layer "F.Cu") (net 4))
 (segment (start 156.8 86.4) (end 156.8 84.6) (width 0.9) (layer "F.Cu") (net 16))
 (via (at 156.8 86.4) (size 0.8) (drill 0.4) (layers "F.Cu" "B.Cu") (free) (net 16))
 (segment (start 161.1 86.5) (end 161 86.4) (width 0.25) (layer "B.Cu") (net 16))
 (segment (start 161 86.4) (end 156.8 86.4) (width 0.25) (layer "B.Cu") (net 16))
 (segment (start 161.1 89.4) (end 161.1 86.5) (width 0.25) (layer "B.Cu") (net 16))
 (segment (start 167.64 93.84) (end 165.54 93.84) (width 0.25) (layer "B.Cu") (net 16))
 (segment (start 165.54 93.84) (end 161.1 89.4) (width 0.25) (layer "B.Cu") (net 16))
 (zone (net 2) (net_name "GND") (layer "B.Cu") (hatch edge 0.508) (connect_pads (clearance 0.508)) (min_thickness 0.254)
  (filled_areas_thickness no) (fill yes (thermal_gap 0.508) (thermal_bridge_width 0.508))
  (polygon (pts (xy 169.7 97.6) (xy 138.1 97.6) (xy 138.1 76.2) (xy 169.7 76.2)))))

